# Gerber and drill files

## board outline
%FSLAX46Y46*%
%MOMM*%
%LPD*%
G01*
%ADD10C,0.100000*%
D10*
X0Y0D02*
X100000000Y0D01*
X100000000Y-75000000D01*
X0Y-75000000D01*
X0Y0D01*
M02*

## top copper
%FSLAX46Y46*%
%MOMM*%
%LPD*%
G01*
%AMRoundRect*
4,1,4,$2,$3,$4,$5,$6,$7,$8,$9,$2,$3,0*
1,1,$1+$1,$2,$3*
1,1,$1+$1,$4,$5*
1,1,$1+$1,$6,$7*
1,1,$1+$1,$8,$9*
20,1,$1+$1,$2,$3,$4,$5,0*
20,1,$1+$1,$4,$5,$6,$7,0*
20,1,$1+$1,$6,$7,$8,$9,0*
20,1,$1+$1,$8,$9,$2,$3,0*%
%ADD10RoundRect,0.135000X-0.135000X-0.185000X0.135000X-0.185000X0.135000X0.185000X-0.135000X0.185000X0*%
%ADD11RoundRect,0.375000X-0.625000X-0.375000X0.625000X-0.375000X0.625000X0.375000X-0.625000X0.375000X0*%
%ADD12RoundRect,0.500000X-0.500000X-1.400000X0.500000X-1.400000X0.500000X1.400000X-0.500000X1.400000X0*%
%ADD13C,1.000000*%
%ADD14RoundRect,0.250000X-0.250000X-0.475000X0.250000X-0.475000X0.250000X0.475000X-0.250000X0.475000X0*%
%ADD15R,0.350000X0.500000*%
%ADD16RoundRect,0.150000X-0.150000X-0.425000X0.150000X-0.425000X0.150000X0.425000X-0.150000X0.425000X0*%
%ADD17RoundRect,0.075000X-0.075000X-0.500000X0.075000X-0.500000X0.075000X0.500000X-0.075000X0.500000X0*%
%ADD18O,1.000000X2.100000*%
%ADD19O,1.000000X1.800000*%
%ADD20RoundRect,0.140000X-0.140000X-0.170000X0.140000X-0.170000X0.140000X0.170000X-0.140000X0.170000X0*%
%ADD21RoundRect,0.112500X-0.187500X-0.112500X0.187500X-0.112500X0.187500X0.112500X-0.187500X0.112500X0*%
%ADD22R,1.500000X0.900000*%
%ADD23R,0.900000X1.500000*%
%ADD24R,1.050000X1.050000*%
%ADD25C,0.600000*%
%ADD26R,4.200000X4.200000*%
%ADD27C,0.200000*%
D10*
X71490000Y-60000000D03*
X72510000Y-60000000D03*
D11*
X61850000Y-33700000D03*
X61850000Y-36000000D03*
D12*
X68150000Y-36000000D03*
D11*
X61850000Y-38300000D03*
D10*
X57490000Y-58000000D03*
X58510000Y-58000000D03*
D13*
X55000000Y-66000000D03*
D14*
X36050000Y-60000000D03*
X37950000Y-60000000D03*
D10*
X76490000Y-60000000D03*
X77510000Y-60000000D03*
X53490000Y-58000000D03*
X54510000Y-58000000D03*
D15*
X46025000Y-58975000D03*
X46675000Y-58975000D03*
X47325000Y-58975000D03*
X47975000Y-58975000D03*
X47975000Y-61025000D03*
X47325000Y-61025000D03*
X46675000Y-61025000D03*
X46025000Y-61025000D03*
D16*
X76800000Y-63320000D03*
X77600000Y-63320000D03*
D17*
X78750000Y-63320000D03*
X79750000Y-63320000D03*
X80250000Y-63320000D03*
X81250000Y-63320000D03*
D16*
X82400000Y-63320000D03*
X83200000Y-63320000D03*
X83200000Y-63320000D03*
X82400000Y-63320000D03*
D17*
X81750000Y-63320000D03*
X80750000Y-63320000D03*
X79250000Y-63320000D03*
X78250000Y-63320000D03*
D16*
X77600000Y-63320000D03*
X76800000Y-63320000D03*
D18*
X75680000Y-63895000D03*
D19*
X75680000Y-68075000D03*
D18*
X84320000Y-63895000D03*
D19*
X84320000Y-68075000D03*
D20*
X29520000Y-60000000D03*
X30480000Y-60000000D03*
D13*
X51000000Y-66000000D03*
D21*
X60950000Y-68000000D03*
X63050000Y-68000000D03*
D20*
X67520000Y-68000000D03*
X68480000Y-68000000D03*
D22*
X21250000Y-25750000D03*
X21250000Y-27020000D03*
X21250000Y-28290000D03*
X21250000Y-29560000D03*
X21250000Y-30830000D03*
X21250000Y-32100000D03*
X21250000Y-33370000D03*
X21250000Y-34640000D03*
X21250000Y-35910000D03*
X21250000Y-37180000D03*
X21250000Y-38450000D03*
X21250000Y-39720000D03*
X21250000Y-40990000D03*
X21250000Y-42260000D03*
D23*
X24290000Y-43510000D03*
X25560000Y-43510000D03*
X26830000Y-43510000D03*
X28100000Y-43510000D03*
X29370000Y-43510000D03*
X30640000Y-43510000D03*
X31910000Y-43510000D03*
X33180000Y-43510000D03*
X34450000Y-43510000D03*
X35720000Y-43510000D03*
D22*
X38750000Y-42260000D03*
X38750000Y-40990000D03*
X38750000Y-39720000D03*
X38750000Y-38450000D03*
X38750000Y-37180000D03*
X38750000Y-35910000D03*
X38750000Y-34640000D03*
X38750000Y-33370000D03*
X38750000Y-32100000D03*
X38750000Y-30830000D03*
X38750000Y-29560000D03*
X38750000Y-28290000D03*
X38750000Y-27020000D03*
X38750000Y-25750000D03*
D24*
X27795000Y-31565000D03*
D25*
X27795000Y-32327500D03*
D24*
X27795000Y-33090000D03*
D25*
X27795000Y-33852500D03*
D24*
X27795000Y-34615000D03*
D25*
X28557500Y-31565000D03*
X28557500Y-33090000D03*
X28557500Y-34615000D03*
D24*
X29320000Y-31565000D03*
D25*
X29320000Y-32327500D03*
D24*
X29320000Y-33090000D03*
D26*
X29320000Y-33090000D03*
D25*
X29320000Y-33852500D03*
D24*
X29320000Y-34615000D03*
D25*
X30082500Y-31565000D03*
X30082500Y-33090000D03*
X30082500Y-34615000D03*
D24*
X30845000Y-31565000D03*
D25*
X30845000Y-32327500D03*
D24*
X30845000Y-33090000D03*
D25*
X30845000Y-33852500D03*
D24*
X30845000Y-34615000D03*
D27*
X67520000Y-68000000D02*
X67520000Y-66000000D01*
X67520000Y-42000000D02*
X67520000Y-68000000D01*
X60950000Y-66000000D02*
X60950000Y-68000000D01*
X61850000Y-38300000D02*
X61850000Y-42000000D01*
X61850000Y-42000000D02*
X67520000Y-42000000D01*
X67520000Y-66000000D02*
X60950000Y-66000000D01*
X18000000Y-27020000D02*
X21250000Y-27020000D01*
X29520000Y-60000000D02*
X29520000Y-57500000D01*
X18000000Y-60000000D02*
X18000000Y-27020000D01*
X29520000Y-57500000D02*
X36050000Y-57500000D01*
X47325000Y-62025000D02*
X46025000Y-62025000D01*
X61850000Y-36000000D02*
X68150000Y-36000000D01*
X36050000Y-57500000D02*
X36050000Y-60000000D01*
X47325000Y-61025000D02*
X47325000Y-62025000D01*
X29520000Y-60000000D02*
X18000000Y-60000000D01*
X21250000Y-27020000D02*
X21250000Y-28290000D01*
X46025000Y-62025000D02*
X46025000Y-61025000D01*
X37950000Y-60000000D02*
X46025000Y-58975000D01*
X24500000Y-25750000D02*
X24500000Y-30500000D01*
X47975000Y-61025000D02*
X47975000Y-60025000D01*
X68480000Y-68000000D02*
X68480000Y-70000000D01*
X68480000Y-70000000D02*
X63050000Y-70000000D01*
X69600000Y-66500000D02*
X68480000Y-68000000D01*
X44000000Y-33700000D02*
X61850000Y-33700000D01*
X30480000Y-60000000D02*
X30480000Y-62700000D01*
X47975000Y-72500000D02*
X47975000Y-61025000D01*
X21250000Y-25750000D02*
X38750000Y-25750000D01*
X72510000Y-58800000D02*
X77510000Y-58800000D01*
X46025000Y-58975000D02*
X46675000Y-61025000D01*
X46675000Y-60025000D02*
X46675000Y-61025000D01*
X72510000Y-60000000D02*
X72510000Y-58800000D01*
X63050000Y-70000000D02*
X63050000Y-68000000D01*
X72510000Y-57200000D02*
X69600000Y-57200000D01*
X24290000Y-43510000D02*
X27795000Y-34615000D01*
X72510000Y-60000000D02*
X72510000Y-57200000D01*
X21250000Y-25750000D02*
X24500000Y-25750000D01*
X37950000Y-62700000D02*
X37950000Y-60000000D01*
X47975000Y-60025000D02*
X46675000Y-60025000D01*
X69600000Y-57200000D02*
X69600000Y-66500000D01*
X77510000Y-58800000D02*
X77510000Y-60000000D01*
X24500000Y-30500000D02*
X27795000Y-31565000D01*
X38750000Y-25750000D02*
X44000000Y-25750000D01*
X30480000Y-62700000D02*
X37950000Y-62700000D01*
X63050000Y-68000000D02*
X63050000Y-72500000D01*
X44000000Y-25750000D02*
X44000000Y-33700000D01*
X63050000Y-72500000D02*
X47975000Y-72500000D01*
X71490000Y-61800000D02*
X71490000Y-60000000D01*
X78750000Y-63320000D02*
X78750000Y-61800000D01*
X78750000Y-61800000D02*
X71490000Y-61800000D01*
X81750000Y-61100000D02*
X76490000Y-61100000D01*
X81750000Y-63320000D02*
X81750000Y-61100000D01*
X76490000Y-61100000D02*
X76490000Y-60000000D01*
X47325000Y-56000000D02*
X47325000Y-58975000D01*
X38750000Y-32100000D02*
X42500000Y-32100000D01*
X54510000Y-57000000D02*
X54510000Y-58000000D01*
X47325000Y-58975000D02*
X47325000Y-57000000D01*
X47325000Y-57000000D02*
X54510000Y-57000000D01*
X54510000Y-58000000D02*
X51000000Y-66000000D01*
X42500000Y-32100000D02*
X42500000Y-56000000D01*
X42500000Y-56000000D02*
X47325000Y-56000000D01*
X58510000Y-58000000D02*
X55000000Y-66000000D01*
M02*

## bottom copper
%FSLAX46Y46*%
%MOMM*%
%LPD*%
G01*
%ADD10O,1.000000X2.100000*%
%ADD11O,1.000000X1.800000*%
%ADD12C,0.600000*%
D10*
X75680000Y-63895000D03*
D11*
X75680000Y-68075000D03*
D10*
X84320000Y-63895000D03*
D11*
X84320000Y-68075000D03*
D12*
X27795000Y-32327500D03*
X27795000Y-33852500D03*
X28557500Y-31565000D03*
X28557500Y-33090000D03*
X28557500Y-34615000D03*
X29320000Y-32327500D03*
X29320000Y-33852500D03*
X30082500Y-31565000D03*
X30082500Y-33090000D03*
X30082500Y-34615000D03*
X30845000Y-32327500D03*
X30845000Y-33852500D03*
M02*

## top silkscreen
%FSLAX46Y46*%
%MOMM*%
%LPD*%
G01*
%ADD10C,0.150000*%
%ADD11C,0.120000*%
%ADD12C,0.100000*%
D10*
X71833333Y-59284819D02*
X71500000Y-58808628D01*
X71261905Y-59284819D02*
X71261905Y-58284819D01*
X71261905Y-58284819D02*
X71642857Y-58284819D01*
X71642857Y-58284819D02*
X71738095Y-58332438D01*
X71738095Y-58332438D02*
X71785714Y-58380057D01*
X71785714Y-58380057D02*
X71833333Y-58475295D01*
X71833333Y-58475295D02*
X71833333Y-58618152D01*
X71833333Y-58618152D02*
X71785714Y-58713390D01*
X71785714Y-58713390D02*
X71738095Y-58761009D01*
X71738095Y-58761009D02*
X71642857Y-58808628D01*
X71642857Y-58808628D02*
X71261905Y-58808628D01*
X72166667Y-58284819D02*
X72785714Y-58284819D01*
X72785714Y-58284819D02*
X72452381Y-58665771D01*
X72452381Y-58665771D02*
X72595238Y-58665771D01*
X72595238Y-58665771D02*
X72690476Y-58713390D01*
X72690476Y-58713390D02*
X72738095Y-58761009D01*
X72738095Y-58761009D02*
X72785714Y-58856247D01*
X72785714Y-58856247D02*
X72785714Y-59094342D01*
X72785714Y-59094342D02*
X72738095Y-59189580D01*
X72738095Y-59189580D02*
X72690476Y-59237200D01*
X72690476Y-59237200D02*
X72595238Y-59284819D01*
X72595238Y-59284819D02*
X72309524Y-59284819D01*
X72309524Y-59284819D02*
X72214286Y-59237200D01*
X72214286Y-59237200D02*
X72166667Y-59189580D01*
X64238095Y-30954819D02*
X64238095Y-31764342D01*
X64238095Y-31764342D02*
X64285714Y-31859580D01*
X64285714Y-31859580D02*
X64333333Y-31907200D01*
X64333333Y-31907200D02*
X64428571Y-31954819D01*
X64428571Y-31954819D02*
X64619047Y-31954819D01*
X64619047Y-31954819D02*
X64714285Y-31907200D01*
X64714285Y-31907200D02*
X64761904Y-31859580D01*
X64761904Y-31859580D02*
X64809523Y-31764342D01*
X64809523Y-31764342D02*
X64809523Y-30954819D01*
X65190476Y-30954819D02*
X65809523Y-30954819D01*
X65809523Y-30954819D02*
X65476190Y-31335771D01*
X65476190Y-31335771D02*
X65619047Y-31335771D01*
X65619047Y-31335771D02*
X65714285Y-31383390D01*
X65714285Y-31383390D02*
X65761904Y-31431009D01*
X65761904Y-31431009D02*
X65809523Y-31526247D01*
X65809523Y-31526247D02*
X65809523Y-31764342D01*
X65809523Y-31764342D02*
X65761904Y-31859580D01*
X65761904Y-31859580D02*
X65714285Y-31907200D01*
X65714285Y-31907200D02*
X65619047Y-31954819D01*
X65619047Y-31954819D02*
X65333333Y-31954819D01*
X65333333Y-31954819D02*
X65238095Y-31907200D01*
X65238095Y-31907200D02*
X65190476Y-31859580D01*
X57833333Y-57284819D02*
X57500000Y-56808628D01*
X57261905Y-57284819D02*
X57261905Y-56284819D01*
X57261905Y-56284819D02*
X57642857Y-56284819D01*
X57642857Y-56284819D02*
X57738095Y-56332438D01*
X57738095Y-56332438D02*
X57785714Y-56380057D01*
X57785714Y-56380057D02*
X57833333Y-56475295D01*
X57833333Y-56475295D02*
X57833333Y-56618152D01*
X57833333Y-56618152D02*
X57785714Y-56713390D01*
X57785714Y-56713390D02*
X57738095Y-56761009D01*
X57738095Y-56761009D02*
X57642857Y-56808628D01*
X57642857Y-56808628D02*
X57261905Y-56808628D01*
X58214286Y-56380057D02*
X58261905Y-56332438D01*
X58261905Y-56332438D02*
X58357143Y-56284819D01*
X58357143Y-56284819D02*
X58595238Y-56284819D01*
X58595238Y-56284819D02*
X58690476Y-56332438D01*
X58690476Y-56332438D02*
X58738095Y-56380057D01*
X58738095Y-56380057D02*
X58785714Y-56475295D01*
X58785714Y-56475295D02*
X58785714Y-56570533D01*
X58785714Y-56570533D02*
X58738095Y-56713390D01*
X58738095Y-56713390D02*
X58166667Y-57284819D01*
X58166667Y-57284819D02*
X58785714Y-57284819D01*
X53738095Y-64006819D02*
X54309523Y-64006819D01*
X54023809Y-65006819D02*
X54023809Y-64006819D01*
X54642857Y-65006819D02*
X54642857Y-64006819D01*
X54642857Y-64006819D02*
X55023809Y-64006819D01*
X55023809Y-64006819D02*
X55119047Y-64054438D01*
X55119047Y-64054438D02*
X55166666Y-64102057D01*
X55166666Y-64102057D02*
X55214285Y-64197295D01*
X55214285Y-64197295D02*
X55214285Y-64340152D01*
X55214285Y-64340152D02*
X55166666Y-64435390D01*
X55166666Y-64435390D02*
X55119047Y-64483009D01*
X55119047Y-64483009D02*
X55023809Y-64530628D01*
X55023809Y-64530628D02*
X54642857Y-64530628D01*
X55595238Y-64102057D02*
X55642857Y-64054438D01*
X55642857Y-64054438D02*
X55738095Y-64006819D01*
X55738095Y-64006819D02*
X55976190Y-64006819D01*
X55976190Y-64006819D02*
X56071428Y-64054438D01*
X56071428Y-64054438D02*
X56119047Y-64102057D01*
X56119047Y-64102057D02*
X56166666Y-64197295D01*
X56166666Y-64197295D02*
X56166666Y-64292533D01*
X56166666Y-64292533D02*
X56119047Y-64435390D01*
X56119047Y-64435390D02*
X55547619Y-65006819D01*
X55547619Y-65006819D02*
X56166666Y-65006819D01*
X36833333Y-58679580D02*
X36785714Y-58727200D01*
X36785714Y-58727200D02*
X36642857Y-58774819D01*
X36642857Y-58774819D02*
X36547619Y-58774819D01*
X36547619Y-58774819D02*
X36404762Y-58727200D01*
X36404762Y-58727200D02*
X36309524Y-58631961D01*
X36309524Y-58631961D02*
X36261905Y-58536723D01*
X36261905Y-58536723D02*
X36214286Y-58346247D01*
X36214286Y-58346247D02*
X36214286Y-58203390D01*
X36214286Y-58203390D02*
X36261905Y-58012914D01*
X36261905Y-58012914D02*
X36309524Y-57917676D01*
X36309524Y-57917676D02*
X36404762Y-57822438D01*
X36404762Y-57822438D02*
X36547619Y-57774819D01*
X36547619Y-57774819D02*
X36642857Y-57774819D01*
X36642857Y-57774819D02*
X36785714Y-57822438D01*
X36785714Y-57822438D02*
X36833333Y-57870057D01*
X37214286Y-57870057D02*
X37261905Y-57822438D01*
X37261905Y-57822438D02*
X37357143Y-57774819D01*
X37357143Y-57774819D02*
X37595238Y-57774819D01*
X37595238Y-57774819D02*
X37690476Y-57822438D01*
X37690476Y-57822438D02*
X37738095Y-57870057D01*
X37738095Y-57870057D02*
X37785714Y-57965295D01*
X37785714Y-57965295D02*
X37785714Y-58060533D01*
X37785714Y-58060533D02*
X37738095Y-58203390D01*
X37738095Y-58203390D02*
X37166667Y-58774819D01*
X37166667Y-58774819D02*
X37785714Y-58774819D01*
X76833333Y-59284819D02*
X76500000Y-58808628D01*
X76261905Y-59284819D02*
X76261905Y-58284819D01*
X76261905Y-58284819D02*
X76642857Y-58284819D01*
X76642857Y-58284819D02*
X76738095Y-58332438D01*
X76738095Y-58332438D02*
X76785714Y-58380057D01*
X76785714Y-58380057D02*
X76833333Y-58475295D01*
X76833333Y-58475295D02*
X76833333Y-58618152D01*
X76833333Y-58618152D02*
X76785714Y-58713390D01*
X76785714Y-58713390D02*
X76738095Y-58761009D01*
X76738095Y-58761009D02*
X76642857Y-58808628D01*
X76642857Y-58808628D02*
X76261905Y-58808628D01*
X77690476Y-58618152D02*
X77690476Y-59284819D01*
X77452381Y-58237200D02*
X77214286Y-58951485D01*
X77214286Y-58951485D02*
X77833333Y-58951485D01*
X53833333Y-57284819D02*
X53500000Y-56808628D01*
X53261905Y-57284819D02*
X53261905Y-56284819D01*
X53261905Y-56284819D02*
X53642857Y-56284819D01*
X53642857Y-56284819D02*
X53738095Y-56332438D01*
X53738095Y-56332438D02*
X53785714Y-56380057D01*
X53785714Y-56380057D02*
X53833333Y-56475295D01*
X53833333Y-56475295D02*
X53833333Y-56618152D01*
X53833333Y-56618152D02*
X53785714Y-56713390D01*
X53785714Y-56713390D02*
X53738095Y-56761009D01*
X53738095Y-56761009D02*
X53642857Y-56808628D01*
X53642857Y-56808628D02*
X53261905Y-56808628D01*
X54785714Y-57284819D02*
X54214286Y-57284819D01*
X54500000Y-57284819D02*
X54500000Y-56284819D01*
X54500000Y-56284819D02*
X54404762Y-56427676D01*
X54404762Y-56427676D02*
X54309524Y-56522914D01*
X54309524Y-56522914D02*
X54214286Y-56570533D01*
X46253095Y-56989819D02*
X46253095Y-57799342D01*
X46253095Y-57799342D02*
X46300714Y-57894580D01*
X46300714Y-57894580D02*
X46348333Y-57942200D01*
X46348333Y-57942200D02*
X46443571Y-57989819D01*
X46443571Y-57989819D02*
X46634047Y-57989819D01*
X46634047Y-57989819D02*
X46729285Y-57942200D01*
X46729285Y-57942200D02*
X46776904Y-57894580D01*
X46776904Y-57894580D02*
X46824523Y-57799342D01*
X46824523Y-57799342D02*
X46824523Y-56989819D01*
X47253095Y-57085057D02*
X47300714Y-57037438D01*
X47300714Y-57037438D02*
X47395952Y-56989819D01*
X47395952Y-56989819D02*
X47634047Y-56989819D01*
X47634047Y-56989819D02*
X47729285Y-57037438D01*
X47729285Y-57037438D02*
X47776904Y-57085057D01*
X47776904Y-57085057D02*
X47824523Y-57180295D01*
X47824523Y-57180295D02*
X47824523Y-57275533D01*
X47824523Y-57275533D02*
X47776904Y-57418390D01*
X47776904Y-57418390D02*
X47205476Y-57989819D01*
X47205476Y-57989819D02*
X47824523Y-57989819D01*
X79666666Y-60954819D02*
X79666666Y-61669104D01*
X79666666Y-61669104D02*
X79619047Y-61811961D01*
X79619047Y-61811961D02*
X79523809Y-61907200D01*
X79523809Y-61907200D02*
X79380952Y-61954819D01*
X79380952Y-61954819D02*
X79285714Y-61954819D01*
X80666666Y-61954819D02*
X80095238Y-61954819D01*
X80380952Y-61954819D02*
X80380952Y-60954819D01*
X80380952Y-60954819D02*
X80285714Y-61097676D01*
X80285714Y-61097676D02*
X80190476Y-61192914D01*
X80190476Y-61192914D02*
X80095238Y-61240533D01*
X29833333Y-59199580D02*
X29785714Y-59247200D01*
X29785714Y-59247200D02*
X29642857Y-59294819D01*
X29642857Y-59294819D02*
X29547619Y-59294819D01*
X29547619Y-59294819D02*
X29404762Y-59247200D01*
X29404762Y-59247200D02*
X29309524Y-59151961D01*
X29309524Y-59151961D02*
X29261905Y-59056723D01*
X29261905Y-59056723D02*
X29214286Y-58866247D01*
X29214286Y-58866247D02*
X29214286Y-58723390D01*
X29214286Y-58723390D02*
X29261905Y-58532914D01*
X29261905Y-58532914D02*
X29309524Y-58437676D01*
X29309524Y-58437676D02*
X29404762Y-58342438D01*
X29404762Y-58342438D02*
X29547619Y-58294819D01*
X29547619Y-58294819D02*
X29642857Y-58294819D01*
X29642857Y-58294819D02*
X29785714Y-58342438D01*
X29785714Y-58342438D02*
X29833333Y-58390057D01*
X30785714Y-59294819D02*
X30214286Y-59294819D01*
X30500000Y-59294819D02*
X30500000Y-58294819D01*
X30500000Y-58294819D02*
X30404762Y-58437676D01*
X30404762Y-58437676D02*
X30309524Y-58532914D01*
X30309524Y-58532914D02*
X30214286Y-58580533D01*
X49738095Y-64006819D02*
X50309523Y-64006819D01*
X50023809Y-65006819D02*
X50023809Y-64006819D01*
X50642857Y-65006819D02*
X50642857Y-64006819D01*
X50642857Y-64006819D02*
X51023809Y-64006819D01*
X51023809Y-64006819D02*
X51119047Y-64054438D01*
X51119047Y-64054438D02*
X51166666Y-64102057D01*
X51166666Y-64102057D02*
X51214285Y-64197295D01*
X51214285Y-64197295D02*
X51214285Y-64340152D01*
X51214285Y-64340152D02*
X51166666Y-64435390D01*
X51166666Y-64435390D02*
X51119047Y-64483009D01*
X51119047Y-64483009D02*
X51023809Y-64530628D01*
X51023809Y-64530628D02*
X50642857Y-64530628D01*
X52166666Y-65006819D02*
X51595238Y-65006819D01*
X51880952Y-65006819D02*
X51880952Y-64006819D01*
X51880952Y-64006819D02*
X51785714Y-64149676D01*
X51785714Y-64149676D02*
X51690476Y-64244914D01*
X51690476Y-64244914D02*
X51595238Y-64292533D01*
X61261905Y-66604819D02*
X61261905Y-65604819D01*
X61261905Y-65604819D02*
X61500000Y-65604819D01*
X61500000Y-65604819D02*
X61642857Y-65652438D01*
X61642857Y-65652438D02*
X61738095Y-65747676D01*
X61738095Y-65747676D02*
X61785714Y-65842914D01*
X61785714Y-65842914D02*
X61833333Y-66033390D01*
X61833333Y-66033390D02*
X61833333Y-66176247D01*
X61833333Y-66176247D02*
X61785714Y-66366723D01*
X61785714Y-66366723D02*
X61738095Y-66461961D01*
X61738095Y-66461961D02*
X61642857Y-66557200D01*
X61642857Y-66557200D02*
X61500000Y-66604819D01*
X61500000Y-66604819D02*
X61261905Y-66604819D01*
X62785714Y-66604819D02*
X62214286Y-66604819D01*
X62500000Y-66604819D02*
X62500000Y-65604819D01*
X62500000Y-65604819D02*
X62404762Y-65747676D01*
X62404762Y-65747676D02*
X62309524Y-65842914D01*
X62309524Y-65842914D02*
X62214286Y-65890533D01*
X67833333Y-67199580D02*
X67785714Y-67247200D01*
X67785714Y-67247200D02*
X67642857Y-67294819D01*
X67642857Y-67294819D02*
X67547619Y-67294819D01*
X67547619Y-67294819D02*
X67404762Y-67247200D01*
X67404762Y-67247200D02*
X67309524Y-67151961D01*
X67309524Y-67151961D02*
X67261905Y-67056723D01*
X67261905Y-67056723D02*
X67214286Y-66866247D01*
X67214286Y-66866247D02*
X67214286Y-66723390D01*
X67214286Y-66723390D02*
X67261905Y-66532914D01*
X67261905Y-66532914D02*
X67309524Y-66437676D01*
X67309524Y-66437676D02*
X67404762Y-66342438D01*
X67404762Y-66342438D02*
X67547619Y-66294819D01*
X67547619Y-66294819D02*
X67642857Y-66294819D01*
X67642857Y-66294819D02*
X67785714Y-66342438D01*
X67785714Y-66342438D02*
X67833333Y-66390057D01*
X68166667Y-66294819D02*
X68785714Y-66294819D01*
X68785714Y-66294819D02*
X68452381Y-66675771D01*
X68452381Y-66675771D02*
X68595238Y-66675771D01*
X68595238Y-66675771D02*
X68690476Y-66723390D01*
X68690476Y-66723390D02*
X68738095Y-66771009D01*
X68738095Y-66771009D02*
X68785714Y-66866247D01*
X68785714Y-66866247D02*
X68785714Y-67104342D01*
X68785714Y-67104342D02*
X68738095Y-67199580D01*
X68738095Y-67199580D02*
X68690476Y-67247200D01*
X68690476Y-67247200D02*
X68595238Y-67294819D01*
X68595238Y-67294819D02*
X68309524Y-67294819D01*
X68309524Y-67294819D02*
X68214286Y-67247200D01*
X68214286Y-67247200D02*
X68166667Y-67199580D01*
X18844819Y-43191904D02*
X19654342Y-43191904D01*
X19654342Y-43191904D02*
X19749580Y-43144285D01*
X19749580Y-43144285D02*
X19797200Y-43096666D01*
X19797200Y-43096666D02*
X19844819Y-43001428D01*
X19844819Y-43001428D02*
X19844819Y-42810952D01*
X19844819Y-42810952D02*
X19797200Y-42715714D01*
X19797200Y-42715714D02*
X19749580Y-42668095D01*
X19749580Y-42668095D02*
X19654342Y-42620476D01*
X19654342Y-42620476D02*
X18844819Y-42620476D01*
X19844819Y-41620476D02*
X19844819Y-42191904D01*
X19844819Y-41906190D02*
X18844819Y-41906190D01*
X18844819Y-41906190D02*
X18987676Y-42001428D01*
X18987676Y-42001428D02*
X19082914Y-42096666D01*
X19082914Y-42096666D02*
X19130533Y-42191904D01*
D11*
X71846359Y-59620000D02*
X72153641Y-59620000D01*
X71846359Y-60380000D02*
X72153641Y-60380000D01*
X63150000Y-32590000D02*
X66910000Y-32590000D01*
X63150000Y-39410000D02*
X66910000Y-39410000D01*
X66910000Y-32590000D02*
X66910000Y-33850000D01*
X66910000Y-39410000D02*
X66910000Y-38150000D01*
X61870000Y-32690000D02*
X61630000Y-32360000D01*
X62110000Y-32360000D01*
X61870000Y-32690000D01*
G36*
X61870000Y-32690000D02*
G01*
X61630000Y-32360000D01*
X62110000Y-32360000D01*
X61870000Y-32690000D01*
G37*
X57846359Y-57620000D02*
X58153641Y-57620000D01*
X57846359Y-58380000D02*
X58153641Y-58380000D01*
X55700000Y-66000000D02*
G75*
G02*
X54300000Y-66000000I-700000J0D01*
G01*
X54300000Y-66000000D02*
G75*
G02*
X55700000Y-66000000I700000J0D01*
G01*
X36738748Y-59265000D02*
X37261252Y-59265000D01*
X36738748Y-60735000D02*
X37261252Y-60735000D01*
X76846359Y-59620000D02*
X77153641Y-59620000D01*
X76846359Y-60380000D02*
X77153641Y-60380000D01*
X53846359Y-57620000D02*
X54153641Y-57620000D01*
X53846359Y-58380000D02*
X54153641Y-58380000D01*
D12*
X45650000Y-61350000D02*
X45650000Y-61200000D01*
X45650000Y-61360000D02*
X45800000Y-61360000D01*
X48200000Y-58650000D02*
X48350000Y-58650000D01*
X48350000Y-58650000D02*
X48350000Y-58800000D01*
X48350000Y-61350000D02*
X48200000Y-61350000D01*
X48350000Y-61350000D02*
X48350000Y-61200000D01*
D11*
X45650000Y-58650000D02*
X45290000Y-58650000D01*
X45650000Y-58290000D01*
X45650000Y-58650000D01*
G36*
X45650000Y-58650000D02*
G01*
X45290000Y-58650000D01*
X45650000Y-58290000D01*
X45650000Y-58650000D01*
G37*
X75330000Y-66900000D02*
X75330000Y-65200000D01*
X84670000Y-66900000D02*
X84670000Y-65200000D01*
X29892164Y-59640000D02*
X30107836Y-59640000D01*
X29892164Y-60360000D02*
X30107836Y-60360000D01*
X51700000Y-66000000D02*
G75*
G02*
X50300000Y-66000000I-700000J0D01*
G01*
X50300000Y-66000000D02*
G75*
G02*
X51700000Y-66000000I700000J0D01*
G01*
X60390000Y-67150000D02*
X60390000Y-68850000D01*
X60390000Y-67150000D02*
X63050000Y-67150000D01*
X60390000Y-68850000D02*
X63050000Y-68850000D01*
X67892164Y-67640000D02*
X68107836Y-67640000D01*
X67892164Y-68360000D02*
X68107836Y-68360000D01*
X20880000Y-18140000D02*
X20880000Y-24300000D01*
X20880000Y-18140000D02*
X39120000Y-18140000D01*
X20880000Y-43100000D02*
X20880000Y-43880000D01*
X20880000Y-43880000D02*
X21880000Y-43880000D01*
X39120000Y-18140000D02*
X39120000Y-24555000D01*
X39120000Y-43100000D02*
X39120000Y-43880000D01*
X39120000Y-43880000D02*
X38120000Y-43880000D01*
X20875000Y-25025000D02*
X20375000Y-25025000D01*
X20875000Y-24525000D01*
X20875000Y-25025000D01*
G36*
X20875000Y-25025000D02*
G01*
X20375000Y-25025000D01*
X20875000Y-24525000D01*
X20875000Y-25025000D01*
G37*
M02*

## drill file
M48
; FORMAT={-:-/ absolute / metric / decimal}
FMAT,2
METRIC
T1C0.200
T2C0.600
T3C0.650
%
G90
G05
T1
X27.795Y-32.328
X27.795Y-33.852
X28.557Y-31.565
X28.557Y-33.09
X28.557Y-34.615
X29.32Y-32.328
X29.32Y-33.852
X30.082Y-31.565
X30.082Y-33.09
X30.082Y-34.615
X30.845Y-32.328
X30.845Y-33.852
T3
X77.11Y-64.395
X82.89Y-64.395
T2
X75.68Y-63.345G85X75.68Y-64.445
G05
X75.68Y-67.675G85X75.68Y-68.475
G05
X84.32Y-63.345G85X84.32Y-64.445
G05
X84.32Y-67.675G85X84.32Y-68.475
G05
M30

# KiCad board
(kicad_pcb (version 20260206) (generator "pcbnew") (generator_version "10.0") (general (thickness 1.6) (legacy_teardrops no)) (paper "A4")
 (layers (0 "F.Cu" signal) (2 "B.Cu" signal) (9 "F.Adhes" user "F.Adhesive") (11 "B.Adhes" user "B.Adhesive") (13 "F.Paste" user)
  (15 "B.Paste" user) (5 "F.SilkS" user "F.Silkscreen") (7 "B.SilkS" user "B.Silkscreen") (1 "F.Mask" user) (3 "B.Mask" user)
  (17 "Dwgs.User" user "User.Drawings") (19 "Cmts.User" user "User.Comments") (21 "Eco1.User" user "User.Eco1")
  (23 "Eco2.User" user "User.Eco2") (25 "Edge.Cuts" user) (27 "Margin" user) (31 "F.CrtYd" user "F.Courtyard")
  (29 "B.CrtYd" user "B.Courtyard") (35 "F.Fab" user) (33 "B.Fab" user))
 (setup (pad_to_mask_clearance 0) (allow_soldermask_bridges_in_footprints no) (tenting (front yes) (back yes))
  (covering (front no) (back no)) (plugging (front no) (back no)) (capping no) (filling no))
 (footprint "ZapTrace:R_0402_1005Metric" (layer "F.Cu") (at 72 60)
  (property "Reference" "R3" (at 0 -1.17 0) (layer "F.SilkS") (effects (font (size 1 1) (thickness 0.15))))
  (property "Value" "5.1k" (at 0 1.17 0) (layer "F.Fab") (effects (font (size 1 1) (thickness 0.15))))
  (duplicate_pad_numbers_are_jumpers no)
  (fp_line (start -0.153641 -0.38) (end 0.153641 -0.38) (stroke (width 0.12) (type solid)) (layer "F.SilkS"))
  (fp_line (start -0.153641 0.38) (end 0.153641 0.38) (stroke (width 0.12) (type solid)) (layer "F.SilkS"))
  (pad "1" smd roundrect (at -0.51 0) (size 0.54 0.64) (layers "F.Cu" "F.Mask" "F.Paste") (roundrect_rratio 0.25) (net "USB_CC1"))
  (pad "2" smd roundrect (at 0.51 0) (size 0.54 0.64) (layers "F.Cu" "F.Mask" "F.Paste") (roundrect_rratio 0.25) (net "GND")))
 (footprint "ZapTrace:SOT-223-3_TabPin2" (layer "F.Cu") (at 65 36)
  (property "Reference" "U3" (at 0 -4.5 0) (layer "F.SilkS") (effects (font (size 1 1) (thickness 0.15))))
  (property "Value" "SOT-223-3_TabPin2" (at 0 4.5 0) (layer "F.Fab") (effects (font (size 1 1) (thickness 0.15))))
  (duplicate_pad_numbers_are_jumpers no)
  (fp_line (start -1.85 -3.41) (end 1.91 -3.41) (stroke (width 0.12) (type solid)) (layer "F.SilkS"))
  (fp_line (start -1.85 3.41) (end 1.91 3.41) (stroke (width 0.12) (type solid)) (layer "F.SilkS"))
  (fp_line (start 1.91 -3.41) (end 1.91 -2.15) (stroke (width 0.12) (type solid)) (layer "F.SilkS"))
  (fp_line (start 1.91 3.41) (end 1.91 2.15) (stroke (width 0.12) (type solid)) (layer "F.SilkS"))
  (fp_poly
   (pts (xy -3.13 -3.31) (xy -3.37 -3.64) (xy -2.89 -3.64) (xy -3.13 -3.31)) (stroke (width 0.12) (type solid)) (fill yes) (layer "F.SilkS"))
  (pad "1" smd roundrect (at -3.15 -2.3) (size 2 1.5) (layers "F.Cu" "F.Mask" "F.Paste") (roundrect_rratio 0.25) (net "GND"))
  (pad "2" smd roundrect (at -3.15 0) (size 2 1.5) (layers "F.Cu" "F.Mask" "F.Paste") (roundrect_rratio 0.25) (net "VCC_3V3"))
  (pad "2" smd roundrect (at 3.15 0) (size 2 3.8) (layers "F.Cu" "F.Mask" "F.Paste") (roundrect_rratio 0.25) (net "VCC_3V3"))
  (pad "3" smd roundrect (at -3.15 2.3) (size 2 1.5) (layers "F.Cu" "F.Mask" "F.Paste") (roundrect_rratio 0.25) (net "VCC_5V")))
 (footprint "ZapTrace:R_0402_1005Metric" (layer "F.Cu") (at 58 58)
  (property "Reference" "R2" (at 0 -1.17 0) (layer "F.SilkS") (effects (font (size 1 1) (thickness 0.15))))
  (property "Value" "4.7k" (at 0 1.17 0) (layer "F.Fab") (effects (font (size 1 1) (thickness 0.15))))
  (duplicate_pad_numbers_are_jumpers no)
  (fp_line (start -0.153641 -0.38) (end 0.153641 -0.38) (stroke (width 0.12) (type solid)) (layer "F.SilkS"))
  (fp_line (start -0.153641 0.38) (end 0.153641 0.38) (stroke (width 0.12) (type solid)) (layer "F.SilkS"))
  (pad "1" smd roundrect (at -0.51 0) (size 0.54 0.64) (layers "F.Cu" "F.Mask" "F.Paste") (roundrect_rratio 0.25) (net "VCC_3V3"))
  (pad "2" smd roundrect (at 0.51 0) (size 0.54 0.64) (layers "F.Cu" "F.Mask" "F.Paste") (roundrect_rratio 0.25) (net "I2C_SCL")))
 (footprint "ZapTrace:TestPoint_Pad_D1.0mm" (layer "F.Cu") (at 55 66)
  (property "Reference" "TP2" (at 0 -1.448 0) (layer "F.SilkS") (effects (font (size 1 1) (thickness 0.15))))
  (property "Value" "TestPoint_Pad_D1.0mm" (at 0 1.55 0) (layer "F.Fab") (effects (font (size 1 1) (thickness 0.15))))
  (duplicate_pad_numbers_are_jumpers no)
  (fp_circle (center 0 0) (end 0 0.7) (stroke (width 0.12) (type solid)) (fill no) (layer "F.SilkS"))
  (pad "1" smd circle (at 0 0) (size 1 1) (layers "F.Cu" "F.Mask") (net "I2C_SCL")))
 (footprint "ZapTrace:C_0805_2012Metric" (layer "F.Cu") (at 37 60)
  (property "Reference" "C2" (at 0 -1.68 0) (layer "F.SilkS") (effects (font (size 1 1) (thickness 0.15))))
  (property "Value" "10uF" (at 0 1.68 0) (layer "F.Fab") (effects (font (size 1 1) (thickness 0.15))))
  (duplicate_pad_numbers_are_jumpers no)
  (fp_line (start -0.261252 -0.735) (end 0.261252 -0.735) (stroke (width 0.12) (type solid)) (layer "F.SilkS"))
  (fp_line (start -0.261252 0.735) (end 0.261252 0.735) (stroke (width 0.12) (type solid)) (layer "F.SilkS"))
  (pad "1" smd roundrect (at -0.95 0) (size 1 1.45) (layers "F.Cu" "F.Mask" "F.Paste") (roundrect_rratio 0.25) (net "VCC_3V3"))
  (pad "2" smd roundrect (at 0.95 0) (size 1 1.45) (layers "F.Cu" "F.Mask" "F.Paste") (roundrect_rratio 0.25) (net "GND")))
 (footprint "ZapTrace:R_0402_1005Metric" (layer "F.Cu") (at 77 60)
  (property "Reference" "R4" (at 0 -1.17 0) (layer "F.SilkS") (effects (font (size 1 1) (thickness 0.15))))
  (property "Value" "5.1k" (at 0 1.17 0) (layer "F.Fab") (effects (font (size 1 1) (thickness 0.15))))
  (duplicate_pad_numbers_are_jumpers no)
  (fp_line (start -0.153641 -0.38) (end 0.153641 -0.38) (stroke (width 0.12) (type solid)) (layer "F.SilkS"))
  (fp_line (start -0.153641 0.38) (end 0.153641 0.38) (stroke (width 0.12) (type solid)) (layer "F.SilkS"))
  (pad "1" smd roundrect (at -0.51 0) (size 0.54 0.64) (layers "F.Cu" "F.Mask" "F.Paste") (roundrect_rratio 0.25) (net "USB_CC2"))
  (pad "2" smd roundrect (at 0.51 0) (size 0.54 0.64) (layers "F.Cu" "F.Mask" "F.Paste") (roundrect_rratio 0.25) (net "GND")))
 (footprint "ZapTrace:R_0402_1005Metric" (layer "F.Cu") (at 54 58)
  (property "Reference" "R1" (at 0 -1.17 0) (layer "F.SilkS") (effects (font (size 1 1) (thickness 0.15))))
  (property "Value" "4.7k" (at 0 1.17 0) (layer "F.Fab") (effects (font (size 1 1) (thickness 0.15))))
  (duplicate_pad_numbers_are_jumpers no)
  (fp_line (start -0.153641 -0.38) (end 0.153641 -0.38) (stroke (width 0.12) (type solid)) (layer "F.SilkS"))
  (fp_line (start -0.153641 0.38) (end 0.153641 0.38) (stroke (width 0.12) (type solid)) (layer "F.SilkS"))
  (pad "1" smd roundrect (at -0.51 0) (size 0.54 0.64) (layers "F.Cu" "F.Mask" "F.Paste") (roundrect_rratio 0.25) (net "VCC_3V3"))
  (pad "2" smd roundrect (at 0.51 0) (size 0.54 0.64) (layers "F.Cu" "F.Mask" "F.Paste") (roundrect_rratio 0.25) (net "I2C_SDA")))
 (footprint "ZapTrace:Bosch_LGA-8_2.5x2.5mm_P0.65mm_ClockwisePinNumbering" (layer "F.Cu") (at 47 60)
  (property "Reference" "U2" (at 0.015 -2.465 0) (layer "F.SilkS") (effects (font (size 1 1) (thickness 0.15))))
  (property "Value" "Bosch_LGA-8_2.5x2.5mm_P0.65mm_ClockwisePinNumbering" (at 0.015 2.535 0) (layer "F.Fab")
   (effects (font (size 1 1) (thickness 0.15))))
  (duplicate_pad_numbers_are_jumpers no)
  (fp_line (start -1.35 1.35) (end -1.35 1.2) (stroke (width 0.1) (type solid)) (layer "F.SilkS"))
  (fp_line (start -1.35 1.36) (end -1.2 1.36) (stroke (width 0.1) (type solid)) (layer "F.SilkS"))
  (fp_line (start 1.2 -1.35) (end 1.35 -1.35) (stroke (width 0.1) (type solid)) (layer "F.SilkS"))
  (fp_line (start 1.35 -1.35) (end 1.35 -1.2) (stroke (width 0.1) (type solid)) (layer "F.SilkS"))
  (fp_line (start 1.35 1.35) (end 1.2 1.35) (stroke (width 0.1) (type solid)) (layer "F.SilkS"))
  (fp_line (start 1.35 1.35) (end 1.35 1.2) (stroke (width 0.1) (type solid)) (layer "F.SilkS"))
  (fp_poly
   (pts (xy -1.35 -1.35) (xy -1.71 -1.35) (xy -1.35 -1.71) (xy -1.35 -1.35)) (stroke (width 0.12) (type solid)) (fill yes) (layer "F.SilkS"))
  (pad "1" smd rect (at -0.975 -1.025 90) (size 0.5 0.35) (layers "F.Cu" "F.Mask" "F.Paste") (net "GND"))
  (pad "2" smd rect (at -0.325 -1.025 90) (size 0.5 0.35) (layers "F.Cu" "F.Mask" "F.Paste") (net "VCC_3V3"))
  (pad "3" smd rect (at 0.325 -1.025 90) (size 0.5 0.35) (layers "F.Cu" "F.Mask" "F.Paste") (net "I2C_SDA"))
  (pad "4" smd rect (at 0.975 -1.025 90) (size 0.5 0.35) (layers "F.Cu" "F.Mask" "F.Paste") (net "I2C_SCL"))
  (pad "5" smd rect (at 0.975 1.025 90) (size 0.5 0.35) (layers "F.Cu" "F.Mask" "F.Paste") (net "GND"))
  (pad "6" smd rect (at 0.325 1.025 90) (size 0.5 0.35) (layers "F.Cu" "F.Mask" "F.Paste") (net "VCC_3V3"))
  (pad "7" smd rect (at -0.325 1.025 90) (size 0.5 0.35) (layers "F.Cu" "F.Mask" "F.Paste") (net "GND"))
  (pad "8" smd rect (at -0.975 1.025 90) (size 0.5 0.35) (layers "F.Cu" "F.Mask" "F.Paste") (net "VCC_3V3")))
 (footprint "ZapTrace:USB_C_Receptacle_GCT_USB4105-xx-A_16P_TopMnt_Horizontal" (layer "F.Cu") (at 80 67)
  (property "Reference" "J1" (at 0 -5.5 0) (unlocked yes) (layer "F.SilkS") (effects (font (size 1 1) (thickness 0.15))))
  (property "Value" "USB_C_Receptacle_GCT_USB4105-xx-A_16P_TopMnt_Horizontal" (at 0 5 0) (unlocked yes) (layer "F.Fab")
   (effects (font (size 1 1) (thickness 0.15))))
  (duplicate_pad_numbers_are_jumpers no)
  (fp_line (start -4.67 -0.1) (end -4.67 -1.8) (stroke (width 0.12) (type solid)) (layer "F.SilkS"))
  (fp_line (start 4.67 -0.1) (end 4.67 -1.8) (stroke (width 0.12) (type solid)) (layer "F.SilkS"))
  (pad "" np_thru_hole circle (at -2.89 -2.605) (size 0.65 0.65) (drill 0.65) (layers "*.Cu" "*.Mask"))
  (pad "" np_thru_hole circle (at 2.89 -2.605) (size 0.65 0.65) (drill 0.65) (layers "*.Cu" "*.Mask"))
  (pad "A1" smd roundrect (at -3.2 -3.68) (size 0.6 1.15) (layers "F.Cu" "F.Mask" "F.Paste") (roundrect_rratio 0.25) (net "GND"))
  (pad "A4" smd roundrect (at -2.4 -3.68) (size 0.6 1.15) (layers "F.Cu" "F.Mask" "F.Paste") (roundrect_rratio 0.25) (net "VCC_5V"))
  (pad "A5" smd roundrect (at -1.25 -3.68) (size 0.3 1.15) (layers "F.Cu" "F.Mask" "F.Paste") (roundrect_rratio 0.25) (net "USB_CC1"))
  (pad "A6" smd roundrect (at -0.25 -3.68) (size 0.3 1.15) (layers "F.Cu" "F.Mask" "F.Paste") (roundrect_rratio 0.25))
  (pad "A7" smd roundrect (at 0.25 -3.68) (size 0.3 1.15) (layers "F.Cu" "F.Mask" "F.Paste") (roundrect_rratio 0.25))
  (pad "A8" smd roundrect (at 1.25 -3.68) (size 0.3 1.15) (layers "F.Cu" "F.Mask" "F.Paste") (roundrect_rratio 0.25))
  (pad "A9" smd roundrect (at 2.4 -3.68) (size 0.6 1.15) (layers "F.Cu" "F.Mask" "F.Paste") (roundrect_rratio 0.25) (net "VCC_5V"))
  (pad "A12" smd roundrect (at 3.2 -3.68) (size 0.6 1.15) (layers "F.Cu" "F.Mask" "F.Paste") (roundrect_rratio 0.25) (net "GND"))
  (pad "B1" smd roundrect (at 3.2 -3.68) (size 0.6 1.15) (layers "F.Cu" "F.Mask" "F.Paste") (roundrect_rratio 0.25) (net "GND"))
  (pad "B4" smd roundrect (at 2.4 -3.68) (size 0.6 1.15) (layers "F.Cu" "F.Mask" "F.Paste") (roundrect_rratio 0.25) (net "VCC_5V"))
  (pad "B5" smd roundrect (at 1.75 -3.68) (size 0.3 1.15) (layers "F.Cu" "F.Mask" "F.Paste") (roundrect_rratio 0.25) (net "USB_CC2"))
  (pad "B6" smd roundrect (at 0.75 -3.68) (size 0.3 1.15) (layers "F.Cu" "F.Mask" "F.Paste") (roundrect_rratio 0.25))
  (pad "B7" smd roundrect (at -0.75 -3.68) (size 0.3 1.15) (layers "F.Cu" "F.Mask" "F.Paste") (roundrect_rratio 0.25))
  (pad "B8" smd roundrect (at -1.75 -3.68) (size 0.3 1.15) (layers "F.Cu" "F.Mask" "F.Paste") (roundrect_rratio 0.25))
  (pad "B9" smd roundrect (at -2.4 -3.68) (size 0.6 1.15) (layers "F.Cu" "F.Mask" "F.Paste") (roundrect_rratio 0.25) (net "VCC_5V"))
  (pad "B12" smd roundrect (at -3.2 -3.68) (size 0.6 1.15) (layers "F.Cu" "F.Mask" "F.Paste") (roundrect_rratio 0.25) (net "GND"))
  (pad "S1" thru_hole oval (at -4.32 -3.105) (size 1 2.1) (drill oval 0.6 1.7) (layers "*.Cu" "*.Mask" "F.Paste") (remove_unused_layers no))
  (pad "S1" thru_hole oval (at -4.32 1.075) (size 1 1.8) (drill oval 0.6 1.4) (layers "*.Cu" "*.Mask" "F.Paste") (remove_unused_layers no))
  (pad "S1" thru_hole oval (at 4.32 -3.105) (size 1 2.1) (drill oval 0.6 1.7) (layers "*.Cu" "*.Mask" "F.Paste") (remove_unused_layers no))
  (pad "S1" thru_hole oval (at 4.32 1.075) (size 1 1.8) (drill oval 0.6 1.4) (layers "*.Cu" "*.Mask" "F.Paste") (remove_unused_layers no)))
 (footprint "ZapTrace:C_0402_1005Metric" (layer "F.Cu") (at 30 60)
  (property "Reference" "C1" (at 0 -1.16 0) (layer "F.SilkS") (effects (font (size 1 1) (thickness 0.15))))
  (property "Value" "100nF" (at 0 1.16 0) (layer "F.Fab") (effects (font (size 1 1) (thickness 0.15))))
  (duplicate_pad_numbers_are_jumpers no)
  (fp_line (start -0.107836 -0.36) (end 0.107836 -0.36) (stroke (width 0.12) (type solid)) (layer "F.SilkS"))
  (fp_line (start -0.107836 0.36) (end 0.107836 0.36) (stroke (width 0.12) (type solid)) (layer "F.SilkS"))
  (pad "1" smd roundrect (at -0.48 0) (size 0.56 0.62) (layers "F.Cu" "F.Mask" "F.Paste") (roundrect_rratio 0.25) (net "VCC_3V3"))
  (pad "2" smd roundrect (at 0.48 0) (size 0.56 0.62) (layers "F.Cu" "F.Mask" "F.Paste") (roundrect_rratio 0.25) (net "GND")))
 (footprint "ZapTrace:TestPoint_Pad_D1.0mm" (layer "F.Cu") (at 51 66)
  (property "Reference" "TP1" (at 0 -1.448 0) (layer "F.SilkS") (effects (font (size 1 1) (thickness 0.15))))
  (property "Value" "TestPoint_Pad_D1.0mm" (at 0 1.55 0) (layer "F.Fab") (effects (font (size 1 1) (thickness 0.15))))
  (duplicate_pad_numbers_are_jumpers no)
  (fp_circle (center 0 0) (end 0 0.7) (stroke (width 0.12) (type solid)) (fill no) (layer "F.SilkS"))
  (pad "1" smd circle (at 0 0) (size 1 1) (layers "F.Cu" "F.Mask") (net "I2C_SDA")))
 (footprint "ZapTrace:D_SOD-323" (layer "F.Cu") (at 62 68)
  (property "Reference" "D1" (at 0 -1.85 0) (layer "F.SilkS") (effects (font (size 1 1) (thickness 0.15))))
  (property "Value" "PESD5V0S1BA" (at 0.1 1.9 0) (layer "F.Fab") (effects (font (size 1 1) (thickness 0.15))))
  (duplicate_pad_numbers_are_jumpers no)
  (fp_line (start -1.61 -0.85) (end -1.61 0.85) (stroke (width 0.12) (type solid)) (layer "F.SilkS"))
  (fp_line (start -1.61 -0.85) (end 1.05 -0.85) (stroke (width 0.12) (type solid)) (layer "F.SilkS"))
  (fp_line (start -1.61 0.85) (end 1.05 0.85) (stroke (width 0.12) (type solid)) (layer "F.SilkS"))
  (pad "1" smd roundrect (at -1.05 0) (size 0.6 0.45) (layers "F.Cu" "F.Mask" "F.Paste") (roundrect_rratio 0.25) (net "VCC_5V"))
  (pad "2" smd roundrect (at 1.05 0) (size 0.6 0.45) (layers "F.Cu" "F.Mask" "F.Paste") (roundrect_rratio 0.25) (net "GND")))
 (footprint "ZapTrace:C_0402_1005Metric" (layer "F.Cu") (at 68 68)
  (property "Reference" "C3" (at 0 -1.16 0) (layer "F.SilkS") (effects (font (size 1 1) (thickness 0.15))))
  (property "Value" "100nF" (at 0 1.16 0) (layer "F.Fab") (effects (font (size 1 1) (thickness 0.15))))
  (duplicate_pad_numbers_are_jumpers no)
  (fp_line (start -0.107836 -0.36) (end 0.107836 -0.36) (stroke (width 0.12) (type solid)) (layer "F.SilkS"))
  (fp_line (start -0.107836 0.36) (end 0.107836 0.36) (stroke (width 0.12) (type solid)) (layer "F.SilkS"))
  (pad "1" smd roundrect (at -0.48 0) (size 0.56 0.62) (layers "F.Cu" "F.Mask" "F.Paste") (roundrect_rratio 0.25) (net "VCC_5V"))
  (pad "2" smd roundrect (at 0.48 0) (size 0.56 0.62) (layers "F.Cu" "F.Mask" "F.Paste") (roundrect_rratio 0.25) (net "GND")))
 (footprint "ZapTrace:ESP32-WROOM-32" (layer "F.Cu") (at 30 34)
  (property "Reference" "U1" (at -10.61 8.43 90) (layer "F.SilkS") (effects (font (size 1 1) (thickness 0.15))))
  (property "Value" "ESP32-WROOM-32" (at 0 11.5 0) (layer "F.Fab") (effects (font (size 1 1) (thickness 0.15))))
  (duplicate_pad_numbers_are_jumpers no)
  (fp_line (start -9.12 -15.86) (end -9.12 -9.7) (stroke (width 0.12) (type solid)) (layer "F.SilkS"))
  (fp_line (start -9.12 -15.86) (end 9.12 -15.86) (stroke (width 0.12) (type solid)) (layer "F.SilkS"))
  (fp_line (start -9.12 9.1) (end -9.12 9.88) (stroke (width 0.12) (type solid)) (layer "F.SilkS"))
  (fp_line (start -9.12 9.88) (end -8.12 9.88) (stroke (width 0.12) (type solid)) (layer "F.SilkS"))
  (fp_line (start 9.12 -15.86) (end 9.12 -9.445) (stroke (width 0.12) (type solid)) (layer "F.SilkS"))
  (fp_line (start 9.12 9.1) (end 9.12 9.88) (stroke (width 0.12) (type solid)) (layer "F.SilkS"))
  (fp_line (start 9.12 9.88) (end 8.12 9.88) (stroke (width 0.12) (type solid)) (layer "F.SilkS"))
  (fp_poly
   (pts (xy -9.125 -8.975) (xy -9.625 -8.975) (xy -9.125 -9.475) (xy -9.125 -8.975)) (stroke (width 0.12) (type solid)) (fill yes)
   (layer "F.SilkS"))
  (pad "1" smd rect (at -8.75 -8.25) (size 1.5 0.9) (layers "F.Cu" "F.Mask" "F.Paste") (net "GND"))
  (pad "2" smd rect (at -8.75 -6.98) (size 1.5 0.9) (layers "F.Cu" "F.Mask" "F.Paste") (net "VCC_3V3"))
  (pad "3" smd rect (at -8.75 -5.71) (size 1.5 0.9) (layers "F.Cu" "F.Mask" "F.Paste") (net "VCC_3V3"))
  (pad "4" smd rect (at -8.75 -4.44) (size 1.5 0.9) (layers "F.Cu" "F.Mask" "F.Paste"))
  (pad "5" smd rect (at -8.75 -3.17) (size 1.5 0.9) (layers "F.Cu" "F.Mask" "F.Paste"))
  (pad "6" smd rect (at -8.75 -1.9) (size 1.5 0.9) (layers "F.Cu" "F.Mask" "F.Paste"))
  (pad "7" smd rect (at -8.75 -0.63) (size 1.5 0.9) (layers "F.Cu" "F.Mask" "F.Paste"))
  (pad "8" smd rect (at -8.75 0.64) (size 1.5 0.9) (layers "F.Cu" "F.Mask" "F.Paste"))
  (pad "9" smd rect (at -8.75 1.91) (size 1.5 0.9) (layers "F.Cu" "F.Mask" "F.Paste"))
  (pad "10" smd rect (at -8.75 3.18) (size 1.5 0.9) (layers "F.Cu" "F.Mask" "F.Paste"))
  (pad "11" smd rect (at -8.75 4.45) (size 1.5 0.9) (layers "F.Cu" "F.Mask" "F.Paste"))
  (pad "12" smd rect (at -8.75 5.72) (size 1.5 0.9) (layers "F.Cu" "F.Mask" "F.Paste"))
  (pad "13" smd rect (at -8.75 6.99) (size 1.5 0.9) (layers "F.Cu" "F.Mask" "F.Paste"))
  (pad "14" smd rect (at -8.75 8.26) (size 1.5 0.9) (layers "F.Cu" "F.Mask" "F.Paste"))
  (pad "15" smd rect (at -5.71 9.51 90) (size 1.5 0.9) (layers "F.Cu" "F.Mask" "F.Paste") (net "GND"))
  (pad "16" smd rect (at -4.44 9.51 90) (size 1.5 0.9) (layers "F.Cu" "F.Mask" "F.Paste"))
  (pad "17" smd rect (at -3.17 9.51 90) (size 1.5 0.9) (layers "F.Cu" "F.Mask" "F.Paste"))
  (pad "18" smd rect (at -1.9 9.51 90) (size 1.5 0.9) (layers "F.Cu" "F.Mask" "F.Paste"))
  (pad "19" smd rect (at -0.63 9.51 90) (size 1.5 0.9) (layers "F.Cu" "F.Mask" "F.Paste"))
  (pad "20" smd rect (at 0.64 9.51 90) (size 1.5 0.9) (layers "F.Cu" "F.Mask" "F.Paste"))
  (pad "21" smd rect (at 1.91 9.51 90) (size 1.5 0.9) (layers "F.Cu" "F.Mask" "F.Paste"))
  (pad "22" smd rect (at 3.18 9.51 90) (size 1.5 0.9) (layers "F.Cu" "F.Mask" "F.Paste"))
  (pad "23" smd rect (at 4.45 9.51 90) (size 1.5 0.9) (layers "F.Cu" "F.Mask" "F.Paste"))
  (pad "24" smd rect (at 5.72 9.51 90) (size 1.5 0.9) (layers "F.Cu" "F.Mask" "F.Paste"))
  (pad "25" smd rect (at 8.75 8.26) (size 1.5 0.9) (layers "F.Cu" "F.Mask" "F.Paste"))
  (pad "26" smd rect (at 8.75 6.99) (size 1.5 0.9) (layers "F.Cu" "F.Mask" "F.Paste"))
  (pad "27" smd rect (at 8.75 5.72) (size 1.5 0.9) (layers "F.Cu" "F.Mask" "F.Paste"))
  (pad "28" smd rect (at 8.75 4.45) (size 1.5 0.9) (layers "F.Cu" "F.Mask" "F.Paste"))
  (pad "29" smd rect (at 8.75 3.18) (size 1.5 0.9) (layers "F.Cu" "F.Mask" "F.Paste"))
  (pad "30" smd rect (at 8.75 1.91) (size 1.5 0.9) (layers "F.Cu" "F.Mask" "F.Paste"))
  (pad "31" smd rect (at 8.75 0.64) (size 1.5 0.9) (layers "F.Cu" "F.Mask" "F.Paste"))
  (pad "32" smd rect (at 8.75 -0.63) (size 1.5 0.9) (layers "F.Cu" "F.Mask" "F.Paste"))
  (pad "33" smd rect (at 8.75 -1.9) (size 1.5 0.9) (layers "F.Cu" "F.Mask" "F.Paste") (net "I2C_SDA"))
  (pad "34" smd rect (at 8.75 -3.17) (size 1.5 0.9) (layers "F.Cu" "F.Mask" "F.Paste"))
  (pad "35" smd rect (at 8.75 -4.44) (size 1.5 0.9) (layers "F.Cu" "F.Mask" "F.Paste"))
  (pad "36" smd rect (at 8.75 -5.71) (size 1.5 0.9) (layers "F.Cu" "F.Mask" "F.Paste") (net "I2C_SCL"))
  (pad "37" smd rect (at 8.75 -6.98) (size 1.5 0.9) (layers "F.Cu" "F.Mask" "F.Paste"))
  (pad "38" smd rect (at 8.75 -8.25) (size 1.5 0.9) (layers "F.Cu" "F.Mask" "F.Paste") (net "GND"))
  (pad "39" smd rect (at -2.205 -2.435) (size 1.05 1.05) (layers "F.Cu" "F.Paste") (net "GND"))
  (pad "39" thru_hole circle (at -2.205 -1.6725) (size 0.6 0.6) (drill 0.2) (layers "*.Cu" "F.Mask") (remove_unused_layers no) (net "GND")
   (zone_connect 2))
  (pad "39" smd rect (at -2.205 -0.91) (size 1.05 1.05) (layers "F.Cu" "F.Paste") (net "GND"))
  (pad "39" thru_hole circle (at -2.205 -0.1475) (size 0.6 0.6) (drill 0.2) (layers "*.Cu" "F.Mask") (remove_unused_layers no) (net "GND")
   (zone_connect 2))
  (pad "39" smd rect (at -2.205 0.615) (size 1.05 1.05) (layers "F.Cu" "F.Paste") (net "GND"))
  (pad "39" thru_hole circle (at -1.4425 -2.435) (size 0.6 0.6) (drill 0.2) (layers "*.Cu" "F.Mask") (remove_unused_layers no) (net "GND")
   (zone_connect 2))
  (pad "39" thru_hole circle (at -1.4425 -0.91) (size 0.6 0.6) (drill 0.2) (layers "*.Cu" "F.Mask") (remove_unused_layers no) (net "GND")
   (zone_connect 2))
  (pad "39" thru_hole circle (at -1.4425 0.615) (size 0.6 0.6) (drill 0.2) (layers "*.Cu" "F.Mask") (remove_unused_layers no) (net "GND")
   (zone_connect 2))
  (pad "39" smd rect (at -0.68 -2.435) (size 1.05 1.05) (layers "F.Cu" "F.Paste") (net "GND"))
  (pad "39" thru_hole circle (at -0.68 -1.6725) (size 0.6 0.6) (drill 0.2) (layers "*.Cu" "F.Mask") (remove_unused_layers no) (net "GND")
   (zone_connect 2))
  (pad "39" smd rect (at -0.68 -0.91) (size 1.05 1.05) (layers "F.Cu" "F.Paste") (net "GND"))
  (pad "39" smd rect (at -0.68 -0.91) (size 4.2 4.2) (layers "F.Cu" "F.Mask") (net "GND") (zone_connect 2))
  (pad "39" thru_hole circle (at -0.68 -0.1475) (size 0.6 0.6) (drill 0.2) (layers "*.Cu" "F.Mask") (remove_unused_layers no) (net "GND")
   (zone_connect 2))
  (pad "39" smd rect (at -0.68 0.615) (size 1.05 1.05) (layers "F.Cu" "F.Paste") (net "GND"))
  (pad "39" thru_hole circle (at 0.0825 -2.435) (size 0.6 0.6) (drill 0.2) (layers "*.Cu" "F.Mask") (remove_unused_layers no) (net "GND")
   (zone_connect 2))
  (pad "39" thru_hole circle (at 0.0825 -0.91) (size 0.6 0.6) (drill 0.2) (layers "*.Cu" "F.Mask") (remove_unused_layers no) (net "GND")
   (zone_connect 2))
  (pad "39" thru_hole circle (at 0.0825 0.615) (size 0.6 0.6) (drill 0.2) (layers "*.Cu" "F.Mask") (remove_unused_layers no) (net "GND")
   (zone_connect 2))
  (pad "39" smd rect (at 0.845 -2.435) (size 1.05 1.05) (layers "F.Cu" "F.Paste") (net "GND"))
  (pad "39" thru_hole circle (at 0.845 -1.6725) (size 0.6 0.6) (drill 0.2) (layers "*.Cu" "F.Mask") (remove_unused_layers no) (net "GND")
   (zone_connect 2))
  (pad "39" smd rect (at 0.845 -0.91) (size 1.05 1.05) (layers "F.Cu" "F.Paste") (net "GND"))
  (pad "39" thru_hole circle (at 0.845 -0.1475) (size 0.6 0.6) (drill 0.2) (layers "*.Cu" "F.Mask") (remove_unused_layers no) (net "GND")
   (zone_connect 2))
  (pad "39" smd rect (at 0.845 0.615) (size 1.05 1.05) (layers "F.Cu" "F.Paste") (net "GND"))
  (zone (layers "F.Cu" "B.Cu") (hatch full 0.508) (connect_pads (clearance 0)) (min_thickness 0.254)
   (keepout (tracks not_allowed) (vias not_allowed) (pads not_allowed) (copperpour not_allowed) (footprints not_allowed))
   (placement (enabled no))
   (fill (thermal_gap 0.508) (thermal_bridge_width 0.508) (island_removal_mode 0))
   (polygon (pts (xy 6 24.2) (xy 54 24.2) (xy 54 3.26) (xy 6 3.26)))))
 (gr_rect (start 0 0) (end 100 75) (stroke (width 0.1) (type default)) (fill no) (layer "Edge.Cuts"))
 (segment (start 67.52 68) (end 67.52 66) (width 0.2) (layer "F.Cu") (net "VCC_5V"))
 (segment (start 67.52 42) (end 67.52 68) (width 0.2) (layer "F.Cu") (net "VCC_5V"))
 (segment (start 60.95 66) (end 60.95 68) (width 0.2) (layer "F.Cu") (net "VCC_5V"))
 (segment (start 61.85 38.3) (end 61.85 42) (width 0.2) (layer "F.Cu") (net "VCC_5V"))
 (segment (start 61.85 42) (end 67.52 42) (width 0.2) (layer "F.Cu") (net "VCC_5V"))
 (segment (start 67.52 66) (end 60.95 66) (width 0.2) (layer "F.Cu") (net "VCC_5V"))
 (segment (start 18 27.02) (end 21.25 27.02) (width 0.2) (layer "F.Cu") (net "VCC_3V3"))
 (segment (start 29.52 60) (end 29.52 57.5) (width 0.2) (layer "F.Cu") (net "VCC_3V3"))
 (segment (start 18 60) (end 18 27.02) (width 0.2) (layer "F.Cu") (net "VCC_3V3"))
 (segment (start 29.52 57.5) (end 36.05 57.5) (width 0.2) (layer "F.Cu") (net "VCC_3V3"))
 (segment (start 47.325 62.025) (end 46.025 62.025) (width 0.2) (layer "F.Cu") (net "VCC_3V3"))
 (segment (start 61.85 36) (end 68.15 36) (width 0.2) (layer "F.Cu") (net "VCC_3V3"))
 (segment (start 36.05 57.5) (end 36.05 60) (width 0.2) (layer "F.Cu") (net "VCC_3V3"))
 (segment (start 47.325 61.025) (end 47.325 62.025) (width 0.2) (layer "F.Cu") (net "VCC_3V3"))
 (segment (start 29.52 60) (end 18 60) (width 0.2) (layer "F.Cu") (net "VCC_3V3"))
 (segment (start 21.25 27.02) (end 21.25 28.29) (width 0.2) (layer "F.Cu") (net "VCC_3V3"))
 (segment (start 46.025 62.025) (end 46.025 61.025) (width 0.2) (layer "F.Cu") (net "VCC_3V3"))
 (segment (start 37.95 60) (end 46.025 58.975) (width 0.2) (layer "F.Cu") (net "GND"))
 (segment (start 24.5 25.75) (end 24.5 30.5) (width 0.2) (layer "F.Cu") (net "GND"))
 (segment (start 47.975 61.025) (end 47.975 60.025) (width 0.2) (layer "F.Cu") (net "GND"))
 (segment (start 68.48 68) (end 68.48 70) (width 0.2) (layer "F.Cu") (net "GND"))
 (segment (start 68.48 70) (end 63.05 70) (width 0.2) (layer "F.Cu") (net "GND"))
 (segment (start 69.6 66.5) (end 68.48 68) (width 0.2) (layer "F.Cu") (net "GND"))
 (segment (start 44 33.7) (end 61.85 33.7) (width 0.2) (layer "F.Cu") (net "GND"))
 (segment (start 30.48 60) (end 30.48 62.7) (width 0.2) (layer "F.Cu") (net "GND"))
 (segment (start 47.975 72.5) (end 47.975 61.025) (width 0.2) (layer "F.Cu") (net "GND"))
 (segment (start 21.25 25.75) (end 38.75 25.75) (width 0.2) (layer "F.Cu") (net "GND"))
 (segment (start 72.51 58.8) (end 77.51 58.8) (width 0.2) (layer "F.Cu") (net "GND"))
 (segment (start 46.025 58.975) (end 46.675 61.025) (width 0.2) (layer "F.Cu") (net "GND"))
 (segment (start 46.675 60.025) (end 46.675 61.025) (width 0.2) (layer "F.Cu") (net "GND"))
 (segment (start 72.51 60) (end 72.51 58.8) (width 0.2) (layer "F.Cu") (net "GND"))
 (segment (start 63.05 70) (end 63.05 68) (width 0.2) (layer "F.Cu") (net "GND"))
 (segment (start 72.51 57.2) (end 69.6 57.2) (width 0.2) (layer "F.Cu") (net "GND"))
 (segment (start 24.29 43.51) (end 27.795 34.615) (width 0.2) (layer "F.Cu") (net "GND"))
 (segment (start 72.51 60) (end 72.51 57.2) (width 0.2) (layer "F.Cu") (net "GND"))
 (segment (start 21.25 25.75) (end 24.5 25.75) (width 0.2) (layer "F.Cu") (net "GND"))
 (segment (start 37.95 62.7) (end 37.95 60) (width 0.2) (layer "F.Cu") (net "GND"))
 (segment (start 47.975 60.025) (end 46.675 60.025) (width 0.2) (layer "F.Cu") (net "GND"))
 (segment (start 69.6 57.2) (end 69.6 66.5) (width 0.2) (layer "F.Cu") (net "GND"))
 (segment (start 77.51 58.8) (end 77.51 60) (width 0.2) (layer "F.Cu") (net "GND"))
 (segment (start 24.5 30.5) (end 27.795 31.565) (width 0.2) (layer "F.Cu") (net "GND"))
 (segment (start 38.75 25.75) (end 44 25.75) (width 0.2) (layer "F.Cu") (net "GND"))
 (segment (start 30.48 62.7) (end 37.95 62.7) (width 0.2) (layer "F.Cu") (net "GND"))
 (segment (start 63.05 68) (end 63.05 72.5) (width 0.2) (layer "F.Cu") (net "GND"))
 (segment (start 44 25.75) (end 44 33.7) (width 0.2) (layer "F.Cu") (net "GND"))
 (segment (start 63.05 72.5) (end 47.975 72.5) (width 0.2) (layer "F.Cu") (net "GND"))
 (segment (start 71.49 61.8) (end 71.49 60) (width 0.2) (layer "F.Cu") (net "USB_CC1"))
 (segment (start 78.75 63.32) (end 78.75 61.8) (width 0.2) (layer "F.Cu") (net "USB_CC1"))
 (segment (start 78.75 61.8) (end 71.49 61.8) (width 0.2) (layer "F.Cu") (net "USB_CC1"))
 (segment (start 81.75 61.1) (end 76.49 61.1) (width 0.2) (layer "F.Cu") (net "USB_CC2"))
 (segment (start 81.75 63.32) (end 81.75 61.1) (width 0.2) (layer "F.Cu") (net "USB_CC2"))
 (segment (start 76.49 61.1) (end 76.49 60) (width 0.2) (layer "F.Cu") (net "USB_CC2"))
 (segment (start 47.325 56) (end 47.325 58.975) (width 0.2) (layer "F.Cu") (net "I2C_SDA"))
 (segment (start 38.75 32.1) (end 42.5 32.1) (width 0.2) (layer "F.Cu") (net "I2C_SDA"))
 (segment (start 54.51 57) (end 54.51 58) (width 0.2) (layer "F.Cu") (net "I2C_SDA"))
 (segment (start 47.325 58.975) (end 47.325 57) (width 0.2) (layer "F.Cu") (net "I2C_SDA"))
 (segment (start 47.325 57) (end 54.51 57) (width 0.2) (layer "F.Cu") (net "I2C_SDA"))
 (segment (start 54.51 58) (end 51 66) (width 0.2) (layer "F.Cu") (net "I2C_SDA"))
 (segment (start 42.5 32.1) (end 42.5 56) (width 0.2) (layer "F.Cu") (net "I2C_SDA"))
 (segment (start 42.5 56) (end 47.325 56) (width 0.2) (layer "F.Cu") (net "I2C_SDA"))
 (segment (start 58.51 58) (end 55 66) (width 0.2) (layer "F.Cu") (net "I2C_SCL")))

